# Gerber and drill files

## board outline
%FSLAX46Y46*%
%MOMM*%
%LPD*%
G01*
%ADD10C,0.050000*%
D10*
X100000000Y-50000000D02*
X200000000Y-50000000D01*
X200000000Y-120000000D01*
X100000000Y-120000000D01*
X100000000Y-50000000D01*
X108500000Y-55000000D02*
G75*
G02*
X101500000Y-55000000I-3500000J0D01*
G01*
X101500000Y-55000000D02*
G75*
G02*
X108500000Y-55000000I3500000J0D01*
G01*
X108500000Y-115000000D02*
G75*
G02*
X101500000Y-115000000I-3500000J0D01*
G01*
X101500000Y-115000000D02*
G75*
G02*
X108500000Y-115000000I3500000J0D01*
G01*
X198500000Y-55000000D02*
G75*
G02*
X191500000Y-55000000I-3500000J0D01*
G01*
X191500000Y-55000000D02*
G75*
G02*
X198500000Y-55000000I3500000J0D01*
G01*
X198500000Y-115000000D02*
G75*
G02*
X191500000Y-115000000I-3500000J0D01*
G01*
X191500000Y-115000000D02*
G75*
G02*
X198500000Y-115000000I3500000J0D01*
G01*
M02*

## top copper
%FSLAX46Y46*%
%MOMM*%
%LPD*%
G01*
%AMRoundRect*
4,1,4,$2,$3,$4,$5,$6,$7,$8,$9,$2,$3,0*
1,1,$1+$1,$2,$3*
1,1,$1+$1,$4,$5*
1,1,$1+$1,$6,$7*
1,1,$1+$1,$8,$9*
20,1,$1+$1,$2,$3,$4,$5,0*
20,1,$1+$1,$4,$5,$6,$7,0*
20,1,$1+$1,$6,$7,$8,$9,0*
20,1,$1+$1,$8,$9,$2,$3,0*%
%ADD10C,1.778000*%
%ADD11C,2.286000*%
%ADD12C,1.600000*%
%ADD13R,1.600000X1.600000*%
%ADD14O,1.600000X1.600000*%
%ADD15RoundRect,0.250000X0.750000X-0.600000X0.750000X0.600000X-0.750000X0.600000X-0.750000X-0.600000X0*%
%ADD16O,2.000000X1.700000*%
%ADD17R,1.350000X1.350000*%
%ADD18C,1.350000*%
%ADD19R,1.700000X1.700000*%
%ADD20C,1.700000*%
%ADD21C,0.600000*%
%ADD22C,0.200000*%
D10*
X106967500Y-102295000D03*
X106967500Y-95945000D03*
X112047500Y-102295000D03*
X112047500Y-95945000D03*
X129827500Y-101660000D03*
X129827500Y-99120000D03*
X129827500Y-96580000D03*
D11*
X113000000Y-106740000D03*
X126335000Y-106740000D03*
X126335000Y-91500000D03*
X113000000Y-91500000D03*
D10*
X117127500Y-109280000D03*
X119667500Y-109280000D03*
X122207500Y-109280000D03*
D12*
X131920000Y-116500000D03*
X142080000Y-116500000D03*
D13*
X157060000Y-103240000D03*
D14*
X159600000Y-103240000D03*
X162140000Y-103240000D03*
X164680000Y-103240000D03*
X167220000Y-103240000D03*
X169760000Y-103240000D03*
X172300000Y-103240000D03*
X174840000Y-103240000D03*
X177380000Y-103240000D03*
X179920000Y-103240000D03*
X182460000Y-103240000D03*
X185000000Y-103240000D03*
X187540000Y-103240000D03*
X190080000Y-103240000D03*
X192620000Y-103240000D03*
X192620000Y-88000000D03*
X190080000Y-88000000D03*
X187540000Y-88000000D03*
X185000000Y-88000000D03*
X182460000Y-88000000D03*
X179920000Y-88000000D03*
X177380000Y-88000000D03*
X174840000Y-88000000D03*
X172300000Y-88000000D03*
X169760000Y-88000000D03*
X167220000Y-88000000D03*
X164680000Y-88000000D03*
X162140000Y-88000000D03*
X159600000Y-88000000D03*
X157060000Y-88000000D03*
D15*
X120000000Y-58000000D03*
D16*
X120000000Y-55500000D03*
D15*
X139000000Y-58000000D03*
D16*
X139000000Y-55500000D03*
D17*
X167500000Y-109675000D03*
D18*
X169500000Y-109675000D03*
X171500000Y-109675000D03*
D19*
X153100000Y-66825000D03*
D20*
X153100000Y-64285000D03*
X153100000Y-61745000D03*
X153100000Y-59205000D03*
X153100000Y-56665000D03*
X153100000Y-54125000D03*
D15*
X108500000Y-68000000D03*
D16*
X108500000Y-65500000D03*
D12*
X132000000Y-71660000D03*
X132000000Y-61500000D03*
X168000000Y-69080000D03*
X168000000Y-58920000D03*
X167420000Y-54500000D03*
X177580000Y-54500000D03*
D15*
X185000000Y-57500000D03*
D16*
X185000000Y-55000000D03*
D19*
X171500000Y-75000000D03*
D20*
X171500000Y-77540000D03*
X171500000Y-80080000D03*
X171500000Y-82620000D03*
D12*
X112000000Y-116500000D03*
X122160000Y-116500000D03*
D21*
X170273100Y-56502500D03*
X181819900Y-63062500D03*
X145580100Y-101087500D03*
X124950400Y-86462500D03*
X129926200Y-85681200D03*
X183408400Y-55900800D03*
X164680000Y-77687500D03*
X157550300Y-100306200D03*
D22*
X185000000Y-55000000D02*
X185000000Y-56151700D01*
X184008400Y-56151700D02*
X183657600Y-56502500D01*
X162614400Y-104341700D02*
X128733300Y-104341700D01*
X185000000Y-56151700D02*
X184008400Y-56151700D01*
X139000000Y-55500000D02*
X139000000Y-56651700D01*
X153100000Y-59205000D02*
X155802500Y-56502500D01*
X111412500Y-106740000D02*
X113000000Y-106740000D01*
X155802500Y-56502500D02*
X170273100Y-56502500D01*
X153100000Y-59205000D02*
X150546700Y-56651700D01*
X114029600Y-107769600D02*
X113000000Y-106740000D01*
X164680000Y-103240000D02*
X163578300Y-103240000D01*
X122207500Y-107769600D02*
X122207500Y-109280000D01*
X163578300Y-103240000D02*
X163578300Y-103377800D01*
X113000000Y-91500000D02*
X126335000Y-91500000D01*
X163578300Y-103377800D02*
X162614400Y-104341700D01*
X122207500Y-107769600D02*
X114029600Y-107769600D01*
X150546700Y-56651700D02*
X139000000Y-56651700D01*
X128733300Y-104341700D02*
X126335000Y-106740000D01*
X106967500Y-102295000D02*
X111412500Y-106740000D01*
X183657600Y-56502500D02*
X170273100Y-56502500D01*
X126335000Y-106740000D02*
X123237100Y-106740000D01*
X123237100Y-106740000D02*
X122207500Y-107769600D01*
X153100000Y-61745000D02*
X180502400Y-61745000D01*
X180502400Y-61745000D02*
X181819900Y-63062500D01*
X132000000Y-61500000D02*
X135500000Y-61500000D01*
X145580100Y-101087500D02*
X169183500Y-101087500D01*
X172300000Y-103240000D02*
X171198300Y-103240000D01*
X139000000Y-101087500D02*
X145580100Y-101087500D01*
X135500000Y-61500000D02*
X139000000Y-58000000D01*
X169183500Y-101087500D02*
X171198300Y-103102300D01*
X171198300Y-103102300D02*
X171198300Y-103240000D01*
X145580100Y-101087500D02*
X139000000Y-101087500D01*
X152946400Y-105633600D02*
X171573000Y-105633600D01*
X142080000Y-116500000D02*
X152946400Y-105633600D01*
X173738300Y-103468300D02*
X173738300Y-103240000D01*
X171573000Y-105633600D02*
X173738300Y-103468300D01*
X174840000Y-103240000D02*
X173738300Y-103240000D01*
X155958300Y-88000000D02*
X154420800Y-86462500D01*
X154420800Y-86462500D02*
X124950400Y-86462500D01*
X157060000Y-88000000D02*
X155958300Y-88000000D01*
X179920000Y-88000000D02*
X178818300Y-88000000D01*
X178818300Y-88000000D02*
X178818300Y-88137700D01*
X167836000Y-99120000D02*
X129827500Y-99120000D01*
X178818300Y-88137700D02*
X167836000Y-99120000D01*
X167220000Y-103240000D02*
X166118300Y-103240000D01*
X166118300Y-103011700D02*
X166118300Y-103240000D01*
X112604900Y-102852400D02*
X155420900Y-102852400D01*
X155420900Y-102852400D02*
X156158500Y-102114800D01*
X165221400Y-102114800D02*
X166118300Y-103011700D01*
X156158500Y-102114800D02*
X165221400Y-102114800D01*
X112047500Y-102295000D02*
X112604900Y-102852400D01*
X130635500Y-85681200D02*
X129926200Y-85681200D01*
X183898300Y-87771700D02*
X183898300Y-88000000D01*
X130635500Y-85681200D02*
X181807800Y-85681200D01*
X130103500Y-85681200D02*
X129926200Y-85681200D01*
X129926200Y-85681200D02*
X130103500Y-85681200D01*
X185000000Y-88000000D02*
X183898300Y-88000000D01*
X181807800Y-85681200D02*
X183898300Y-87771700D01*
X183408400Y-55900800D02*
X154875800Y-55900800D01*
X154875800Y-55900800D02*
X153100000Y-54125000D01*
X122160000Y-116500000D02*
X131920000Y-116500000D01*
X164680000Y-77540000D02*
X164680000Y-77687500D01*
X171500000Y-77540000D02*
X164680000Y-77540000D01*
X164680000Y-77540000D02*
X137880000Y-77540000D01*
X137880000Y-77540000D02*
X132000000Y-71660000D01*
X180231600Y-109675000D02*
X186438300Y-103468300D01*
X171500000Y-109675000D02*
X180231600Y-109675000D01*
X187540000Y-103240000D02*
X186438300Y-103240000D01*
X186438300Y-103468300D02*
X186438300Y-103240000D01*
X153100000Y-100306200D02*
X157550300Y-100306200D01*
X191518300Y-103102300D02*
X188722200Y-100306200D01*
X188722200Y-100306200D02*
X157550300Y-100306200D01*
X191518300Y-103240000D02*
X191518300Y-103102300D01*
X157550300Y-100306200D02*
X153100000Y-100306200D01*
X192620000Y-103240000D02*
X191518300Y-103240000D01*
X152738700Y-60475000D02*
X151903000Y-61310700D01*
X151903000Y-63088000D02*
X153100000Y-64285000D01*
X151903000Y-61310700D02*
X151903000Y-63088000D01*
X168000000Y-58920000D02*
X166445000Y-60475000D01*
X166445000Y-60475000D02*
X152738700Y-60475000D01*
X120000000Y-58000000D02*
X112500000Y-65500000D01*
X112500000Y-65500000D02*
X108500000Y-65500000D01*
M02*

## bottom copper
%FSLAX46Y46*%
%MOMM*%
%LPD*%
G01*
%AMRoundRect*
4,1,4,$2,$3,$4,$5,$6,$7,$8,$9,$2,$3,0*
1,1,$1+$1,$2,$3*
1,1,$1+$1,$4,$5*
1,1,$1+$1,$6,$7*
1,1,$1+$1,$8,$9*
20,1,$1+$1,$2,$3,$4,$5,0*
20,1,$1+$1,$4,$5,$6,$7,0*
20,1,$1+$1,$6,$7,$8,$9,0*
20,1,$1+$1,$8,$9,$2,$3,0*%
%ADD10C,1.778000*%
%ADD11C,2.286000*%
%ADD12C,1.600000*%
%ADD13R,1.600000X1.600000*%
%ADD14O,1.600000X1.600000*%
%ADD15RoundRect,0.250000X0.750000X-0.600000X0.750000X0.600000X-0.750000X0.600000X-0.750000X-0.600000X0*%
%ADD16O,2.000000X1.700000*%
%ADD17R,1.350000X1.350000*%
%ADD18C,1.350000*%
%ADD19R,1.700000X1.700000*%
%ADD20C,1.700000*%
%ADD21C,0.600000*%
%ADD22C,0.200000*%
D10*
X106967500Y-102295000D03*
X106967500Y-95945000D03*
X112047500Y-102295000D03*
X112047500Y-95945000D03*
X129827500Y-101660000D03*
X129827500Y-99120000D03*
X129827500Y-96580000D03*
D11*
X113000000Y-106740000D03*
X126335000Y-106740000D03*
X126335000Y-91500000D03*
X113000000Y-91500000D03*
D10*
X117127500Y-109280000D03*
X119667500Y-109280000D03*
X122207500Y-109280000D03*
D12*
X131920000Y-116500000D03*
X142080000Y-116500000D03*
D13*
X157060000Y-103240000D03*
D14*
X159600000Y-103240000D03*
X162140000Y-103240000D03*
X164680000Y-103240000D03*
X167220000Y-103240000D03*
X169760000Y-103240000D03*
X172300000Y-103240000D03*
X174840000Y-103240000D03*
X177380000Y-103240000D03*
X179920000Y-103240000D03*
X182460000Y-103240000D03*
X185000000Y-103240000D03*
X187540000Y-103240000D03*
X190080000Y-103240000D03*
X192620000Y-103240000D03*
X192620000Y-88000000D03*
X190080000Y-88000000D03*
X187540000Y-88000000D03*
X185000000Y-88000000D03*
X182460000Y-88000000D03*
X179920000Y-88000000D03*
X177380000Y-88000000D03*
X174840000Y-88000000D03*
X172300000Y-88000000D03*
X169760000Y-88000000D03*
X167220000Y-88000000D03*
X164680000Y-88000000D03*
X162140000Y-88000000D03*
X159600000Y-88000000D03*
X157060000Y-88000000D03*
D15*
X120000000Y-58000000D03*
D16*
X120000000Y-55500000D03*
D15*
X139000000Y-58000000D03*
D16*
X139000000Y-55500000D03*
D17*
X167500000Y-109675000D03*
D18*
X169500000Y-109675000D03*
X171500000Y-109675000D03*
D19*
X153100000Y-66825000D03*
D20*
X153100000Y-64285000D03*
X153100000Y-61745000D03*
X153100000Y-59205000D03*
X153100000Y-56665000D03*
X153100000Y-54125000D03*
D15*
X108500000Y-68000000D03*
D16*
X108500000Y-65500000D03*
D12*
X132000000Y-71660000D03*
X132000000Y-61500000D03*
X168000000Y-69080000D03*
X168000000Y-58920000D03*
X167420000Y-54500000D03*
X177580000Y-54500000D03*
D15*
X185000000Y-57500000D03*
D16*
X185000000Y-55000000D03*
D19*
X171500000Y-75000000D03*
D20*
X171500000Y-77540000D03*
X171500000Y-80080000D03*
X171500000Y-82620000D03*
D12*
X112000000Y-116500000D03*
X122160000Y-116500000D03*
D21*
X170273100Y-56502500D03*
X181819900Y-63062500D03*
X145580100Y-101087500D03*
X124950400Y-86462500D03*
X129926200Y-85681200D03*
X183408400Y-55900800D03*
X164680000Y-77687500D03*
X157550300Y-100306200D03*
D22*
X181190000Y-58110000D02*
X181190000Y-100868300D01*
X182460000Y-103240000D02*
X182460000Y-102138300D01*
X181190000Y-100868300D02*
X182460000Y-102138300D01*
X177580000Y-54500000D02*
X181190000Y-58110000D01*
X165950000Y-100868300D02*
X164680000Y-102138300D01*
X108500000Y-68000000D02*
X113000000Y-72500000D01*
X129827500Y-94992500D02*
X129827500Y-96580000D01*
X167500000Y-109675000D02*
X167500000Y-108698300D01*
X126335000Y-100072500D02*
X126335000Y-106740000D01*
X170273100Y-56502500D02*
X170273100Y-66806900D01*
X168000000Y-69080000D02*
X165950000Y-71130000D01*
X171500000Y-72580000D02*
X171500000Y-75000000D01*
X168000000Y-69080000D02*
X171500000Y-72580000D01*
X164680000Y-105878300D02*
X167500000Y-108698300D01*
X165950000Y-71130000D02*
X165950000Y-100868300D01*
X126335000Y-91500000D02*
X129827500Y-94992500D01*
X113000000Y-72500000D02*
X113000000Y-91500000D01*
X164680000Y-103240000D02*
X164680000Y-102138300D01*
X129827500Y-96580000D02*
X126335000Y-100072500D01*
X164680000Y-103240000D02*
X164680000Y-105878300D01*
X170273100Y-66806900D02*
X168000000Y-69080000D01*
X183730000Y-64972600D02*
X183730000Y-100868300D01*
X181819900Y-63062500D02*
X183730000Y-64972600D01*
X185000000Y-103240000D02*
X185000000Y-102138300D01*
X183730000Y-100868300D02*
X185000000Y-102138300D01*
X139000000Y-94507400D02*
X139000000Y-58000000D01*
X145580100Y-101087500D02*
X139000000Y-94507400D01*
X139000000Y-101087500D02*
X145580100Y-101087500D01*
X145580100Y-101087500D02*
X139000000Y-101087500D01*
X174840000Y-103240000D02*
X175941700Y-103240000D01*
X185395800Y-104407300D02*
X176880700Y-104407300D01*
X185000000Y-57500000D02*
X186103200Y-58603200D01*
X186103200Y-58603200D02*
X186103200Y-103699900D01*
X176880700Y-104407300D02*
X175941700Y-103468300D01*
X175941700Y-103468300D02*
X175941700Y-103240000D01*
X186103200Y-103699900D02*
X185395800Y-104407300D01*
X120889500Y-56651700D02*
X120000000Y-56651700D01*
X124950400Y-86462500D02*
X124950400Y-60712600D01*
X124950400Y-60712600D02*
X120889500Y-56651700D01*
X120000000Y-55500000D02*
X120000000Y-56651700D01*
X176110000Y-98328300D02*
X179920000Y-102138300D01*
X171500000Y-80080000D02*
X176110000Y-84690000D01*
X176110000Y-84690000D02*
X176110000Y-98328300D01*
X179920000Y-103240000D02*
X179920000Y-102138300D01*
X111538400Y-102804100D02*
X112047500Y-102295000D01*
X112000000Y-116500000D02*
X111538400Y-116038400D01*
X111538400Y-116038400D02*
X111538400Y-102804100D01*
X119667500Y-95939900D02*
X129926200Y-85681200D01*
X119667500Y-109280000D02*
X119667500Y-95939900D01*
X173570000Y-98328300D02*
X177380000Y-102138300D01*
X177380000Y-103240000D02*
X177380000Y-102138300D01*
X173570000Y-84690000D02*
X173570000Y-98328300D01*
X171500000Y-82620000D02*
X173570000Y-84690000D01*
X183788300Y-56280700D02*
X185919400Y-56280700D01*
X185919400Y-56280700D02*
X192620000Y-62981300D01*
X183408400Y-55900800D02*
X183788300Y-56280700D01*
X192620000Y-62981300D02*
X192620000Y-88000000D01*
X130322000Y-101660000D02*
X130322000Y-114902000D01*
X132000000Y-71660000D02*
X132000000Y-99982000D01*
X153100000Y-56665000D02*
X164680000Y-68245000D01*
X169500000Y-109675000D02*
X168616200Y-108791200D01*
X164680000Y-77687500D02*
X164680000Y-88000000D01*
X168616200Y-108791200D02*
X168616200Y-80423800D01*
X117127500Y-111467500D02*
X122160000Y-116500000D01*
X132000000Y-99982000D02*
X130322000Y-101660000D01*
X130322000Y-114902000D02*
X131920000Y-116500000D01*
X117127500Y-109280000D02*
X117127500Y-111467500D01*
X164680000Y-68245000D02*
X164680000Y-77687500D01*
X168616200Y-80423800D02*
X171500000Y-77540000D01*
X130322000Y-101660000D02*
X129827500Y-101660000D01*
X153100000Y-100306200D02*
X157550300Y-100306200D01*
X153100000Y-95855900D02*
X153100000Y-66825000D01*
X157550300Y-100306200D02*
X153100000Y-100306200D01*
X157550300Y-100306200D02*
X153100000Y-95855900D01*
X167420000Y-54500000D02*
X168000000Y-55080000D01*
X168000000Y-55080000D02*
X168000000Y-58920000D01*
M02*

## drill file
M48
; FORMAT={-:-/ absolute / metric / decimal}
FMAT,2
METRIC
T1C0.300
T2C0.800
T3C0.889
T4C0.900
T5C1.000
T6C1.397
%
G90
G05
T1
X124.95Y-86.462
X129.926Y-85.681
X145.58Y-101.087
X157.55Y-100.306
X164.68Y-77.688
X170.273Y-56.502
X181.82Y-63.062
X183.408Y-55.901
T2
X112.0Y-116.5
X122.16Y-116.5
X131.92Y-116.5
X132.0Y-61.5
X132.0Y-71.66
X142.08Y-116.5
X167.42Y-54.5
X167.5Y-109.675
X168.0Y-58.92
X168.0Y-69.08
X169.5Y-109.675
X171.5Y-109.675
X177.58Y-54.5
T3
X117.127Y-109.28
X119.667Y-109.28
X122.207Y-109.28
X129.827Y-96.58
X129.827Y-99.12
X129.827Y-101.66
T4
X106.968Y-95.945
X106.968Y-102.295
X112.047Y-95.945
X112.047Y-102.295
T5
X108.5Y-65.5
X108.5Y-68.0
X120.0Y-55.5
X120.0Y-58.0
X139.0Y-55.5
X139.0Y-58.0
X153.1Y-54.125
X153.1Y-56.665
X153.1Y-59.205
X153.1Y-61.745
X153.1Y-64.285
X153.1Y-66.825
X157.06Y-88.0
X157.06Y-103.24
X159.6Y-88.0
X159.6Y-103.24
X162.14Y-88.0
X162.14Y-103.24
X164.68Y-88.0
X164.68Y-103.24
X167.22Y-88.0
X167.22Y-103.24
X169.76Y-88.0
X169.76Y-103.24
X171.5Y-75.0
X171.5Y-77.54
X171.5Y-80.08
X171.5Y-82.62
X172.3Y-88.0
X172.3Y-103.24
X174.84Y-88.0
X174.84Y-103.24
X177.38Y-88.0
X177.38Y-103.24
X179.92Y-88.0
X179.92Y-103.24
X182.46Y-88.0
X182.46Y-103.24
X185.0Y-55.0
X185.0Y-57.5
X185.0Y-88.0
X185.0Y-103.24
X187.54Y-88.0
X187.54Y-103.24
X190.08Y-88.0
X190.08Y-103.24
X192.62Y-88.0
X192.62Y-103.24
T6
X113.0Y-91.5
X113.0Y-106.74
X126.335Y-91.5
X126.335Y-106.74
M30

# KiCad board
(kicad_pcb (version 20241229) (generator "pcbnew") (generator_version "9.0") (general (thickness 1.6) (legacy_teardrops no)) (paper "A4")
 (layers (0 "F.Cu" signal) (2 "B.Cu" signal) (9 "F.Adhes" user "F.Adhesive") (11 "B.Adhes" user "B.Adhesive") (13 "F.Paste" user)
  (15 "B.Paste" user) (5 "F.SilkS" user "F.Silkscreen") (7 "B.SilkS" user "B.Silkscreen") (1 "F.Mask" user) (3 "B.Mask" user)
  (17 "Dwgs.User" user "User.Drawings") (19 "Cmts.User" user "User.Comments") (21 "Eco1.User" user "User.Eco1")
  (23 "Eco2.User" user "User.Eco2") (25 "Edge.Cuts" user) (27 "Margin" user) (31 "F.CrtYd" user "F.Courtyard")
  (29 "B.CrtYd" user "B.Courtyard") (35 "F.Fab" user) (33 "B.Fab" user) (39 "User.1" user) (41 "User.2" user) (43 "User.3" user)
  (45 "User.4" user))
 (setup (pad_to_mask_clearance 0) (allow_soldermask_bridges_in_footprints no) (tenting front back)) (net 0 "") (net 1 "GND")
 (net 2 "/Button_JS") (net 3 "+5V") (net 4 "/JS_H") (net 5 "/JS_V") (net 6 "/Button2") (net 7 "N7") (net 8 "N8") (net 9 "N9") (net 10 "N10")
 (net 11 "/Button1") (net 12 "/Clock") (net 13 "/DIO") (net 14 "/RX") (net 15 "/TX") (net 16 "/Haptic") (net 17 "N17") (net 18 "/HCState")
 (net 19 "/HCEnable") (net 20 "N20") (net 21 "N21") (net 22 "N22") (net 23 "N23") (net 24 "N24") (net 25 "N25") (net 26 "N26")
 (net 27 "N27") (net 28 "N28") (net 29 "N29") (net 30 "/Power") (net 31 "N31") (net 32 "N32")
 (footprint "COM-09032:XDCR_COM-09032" (layer "F.Cu") (at 119.6675 99.12 90)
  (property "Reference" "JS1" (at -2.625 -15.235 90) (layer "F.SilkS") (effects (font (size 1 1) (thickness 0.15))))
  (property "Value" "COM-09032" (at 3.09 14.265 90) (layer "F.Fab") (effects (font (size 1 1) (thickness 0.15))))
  (pad "B1A" thru_hole circle (at -3.175 -12.7 90) (size 1.778 1.778) (drill 0.9) (layers "*.Cu" "*.Mask") (remove_unused_layers no)
   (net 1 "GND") (solder_mask_margin 0.102))
  (pad "B1B" thru_hole circle (at 3.175 -12.7 90) (size 1.778 1.778) (drill 0.9) (layers "*.Cu" "*.Mask") (remove_unused_layers no)
   (solder_mask_margin 0.102))
  (pad "B2A" thru_hole circle (at -3.175 -7.62 90) (size 1.778 1.778) (drill 0.9) (layers "*.Cu" "*.Mask") (remove_unused_layers no)
   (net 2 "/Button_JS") (solder_mask_margin 0.102))
  (pad "B2B" thru_hole circle (at 3.175 -7.62 90) (size 1.778 1.778) (drill 0.9) (layers "*.Cu" "*.Mask") (remove_unused_layers no)
   (solder_mask_margin 0.102))
  (pad "H1" thru_hole circle (at -2.54 10.16 90) (size 1.778 1.778) (drill 0.889) (layers "*.Cu" "*.Mask") (remove_unused_layers no)
   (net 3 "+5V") (solder_mask_margin 0.102))
  (pad "H2" thru_hole circle (at 0 10.16 90) (size 1.778 1.778) (drill 0.889) (layers "*.Cu" "*.Mask") (remove_unused_layers no)
   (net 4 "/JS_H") (solder_mask_margin 0.102))
  (pad "H3" thru_hole circle (at 2.54 10.16 90) (size 1.778 1.778) (drill 0.889) (layers "*.Cu" "*.Mask") (remove_unused_layers no)
   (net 1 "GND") (solder_mask_margin 0.102))
  (pad "S1" thru_hole circle (at -7.62 -6.6675 90) (size 2.286 2.286) (drill 1.397) (layers "*.Cu" "*.Mask") (remove_unused_layers no)
   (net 1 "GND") (solder_mask_margin 0.102))
  (pad "S2" thru_hole circle (at -7.62 6.6675 90) (size 2.286 2.286) (drill 1.397) (layers "*.Cu" "*.Mask") (remove_unused_layers no)
   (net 1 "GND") (solder_mask_margin 0.102))
  (pad "S3" thru_hole circle (at 7.62 6.6675 90) (size 2.286 2.286) (drill 1.397) (layers "*.Cu" "*.Mask") (remove_unused_layers no)
   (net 1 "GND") (solder_mask_margin 0.102))
  (pad "S4" thru_hole circle (at 7.62 -6.6675 90) (size 2.286 2.286) (drill 1.397) (layers "*.Cu" "*.Mask") (remove_unused_layers no)
   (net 1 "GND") (solder_mask_margin 0.102))
  (pad "V1" thru_hole circle (at -10.16 -2.54 90) (size 1.778 1.778) (drill 0.889) (layers "*.Cu" "*.Mask") (remove_unused_layers no)
   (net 3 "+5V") (solder_mask_margin 0.102))
  (pad "V2" thru_hole circle (at -10.16 0 90) (size 1.778 1.778) (drill 0.889) (layers "*.Cu" "*.Mask") (remove_unused_layers no)
   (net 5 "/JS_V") (solder_mask_margin 0.102))
  (pad "V3" thru_hole circle (at -10.16 2.54 90) (size 1.778 1.778) (drill 0.889) (layers "*.Cu" "*.Mask") (remove_unused_layers no)
   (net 1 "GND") (solder_mask_margin 0.102)))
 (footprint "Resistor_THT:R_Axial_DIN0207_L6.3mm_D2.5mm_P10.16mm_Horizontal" (layer "F.Cu") (at 131.92 116.5)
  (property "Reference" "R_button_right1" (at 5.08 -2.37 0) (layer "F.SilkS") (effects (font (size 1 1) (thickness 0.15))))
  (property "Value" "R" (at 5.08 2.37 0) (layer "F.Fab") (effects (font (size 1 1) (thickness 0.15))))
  (pad "1" thru_hole circle (at 0 0) (size 1.6 1.6) (drill 0.8) (layers "*.Cu" "*.Mask") (remove_unused_layers no) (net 3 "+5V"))
  (pad "2" thru_hole circle (at 10.16 0) (size 1.6 1.6) (drill 0.8) (layers "*.Cu" "*.Mask") (remove_unused_layers no) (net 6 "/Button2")))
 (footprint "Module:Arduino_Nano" (layer "F.Cu") (at 157.06 103.24 90)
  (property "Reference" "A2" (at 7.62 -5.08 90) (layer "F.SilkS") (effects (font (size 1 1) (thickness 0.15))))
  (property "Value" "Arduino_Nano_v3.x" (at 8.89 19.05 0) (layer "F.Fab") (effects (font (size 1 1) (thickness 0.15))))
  (pad "1" thru_hole rect (at 0 0 90) (size 1.6 1.6) (drill 1) (layers "*.Cu" "*.Mask") (remove_unused_layers no) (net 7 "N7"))
  (pad "2" thru_hole oval (at 0 2.54 90) (size 1.6 1.6) (drill 1) (layers "*.Cu" "*.Mask") (remove_unused_layers no) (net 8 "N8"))
  (pad "3" thru_hole oval (at 0 5.08 90) (size 1.6 1.6) (drill 1) (layers "*.Cu" "*.Mask") (remove_unused_layers no) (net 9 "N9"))
  (pad "4" thru_hole oval (at 0 7.62 90) (size 1.6 1.6) (drill 1) (layers "*.Cu" "*.Mask") (remove_unused_layers no) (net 1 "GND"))
  (pad "5" thru_hole oval (at 0 10.16 90) (size 1.6 1.6) (drill 1) (layers "*.Cu" "*.Mask") (remove_unused_layers no) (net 2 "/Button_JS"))
  (pad "6" thru_hole oval (at 0 12.7 90) (size 1.6 1.6) (drill 1) (layers "*.Cu" "*.Mask") (remove_unused_layers no) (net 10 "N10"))
  (pad "7" thru_hole oval (at 0 15.24 90) (size 1.6 1.6) (drill 1) (layers "*.Cu" "*.Mask") (remove_unused_layers no) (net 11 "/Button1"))
  (pad "8" thru_hole oval (at 0 17.78 90) (size 1.6 1.6) (drill 1) (layers "*.Cu" "*.Mask") (remove_unused_layers no) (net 6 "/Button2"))
  (pad "9" thru_hole oval (at 0 20.32 90) (size 1.6 1.6) (drill 1) (layers "*.Cu" "*.Mask") (remove_unused_layers no) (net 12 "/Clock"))
  (pad "10" thru_hole oval (at 0 22.86 90) (size 1.6 1.6) (drill 1) (layers "*.Cu" "*.Mask") (remove_unused_layers no) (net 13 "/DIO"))
  (pad "11" thru_hole oval (at 0 25.4 90) (size 1.6 1.6) (drill 1) (layers "*.Cu" "*.Mask") (remove_unused_layers no) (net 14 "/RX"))
  (pad "12" thru_hole oval (at 0 27.94 90) (size 1.6 1.6) (drill 1) (layers "*.Cu" "*.Mask") (remove_unused_layers no) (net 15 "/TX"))
  (pad "13" thru_hole oval (at 0 30.48 90) (size 1.6 1.6) (drill 1) (layers "*.Cu" "*.Mask") (remove_unused_layers no) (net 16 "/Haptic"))
  (pad "14" thru_hole oval (at 0 33.02 90) (size 1.6 1.6) (drill 1) (layers "*.Cu" "*.Mask") (remove_unused_layers no) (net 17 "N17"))
  (pad "15" thru_hole oval (at 0 35.56 90) (size 1.6 1.6) (drill 1) (layers "*.Cu" "*.Mask") (remove_unused_layers no) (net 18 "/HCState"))
  (pad "16" thru_hole oval (at 15.24 35.56 90) (size 1.6 1.6) (drill 1) (layers "*.Cu" "*.Mask") (remove_unused_layers no)
   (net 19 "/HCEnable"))
  (pad "17" thru_hole oval (at 15.24 33.02 90) (size 1.6 1.6) (drill 1) (layers "*.Cu" "*.Mask") (remove_unused_layers no) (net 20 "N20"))
  (pad "18" thru_hole oval (at 15.24 30.48 90) (size 1.6 1.6) (drill 1) (layers "*.Cu" "*.Mask") (remove_unused_layers no) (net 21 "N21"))
  (pad "19" thru_hole oval (at 15.24 27.94 90) (size 1.6 1.6) (drill 1) (layers "*.Cu" "*.Mask") (remove_unused_layers no) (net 5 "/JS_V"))
  (pad "20" thru_hole oval (at 15.24 25.4 90) (size 1.6 1.6) (drill 1) (layers "*.Cu" "*.Mask") (remove_unused_layers no) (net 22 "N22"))
  (pad "21" thru_hole oval (at 15.24 22.86 90) (size 1.6 1.6) (drill 1) (layers "*.Cu" "*.Mask") (remove_unused_layers no) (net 4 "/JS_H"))
  (pad "22" thru_hole oval (at 15.24 20.32 90) (size 1.6 1.6) (drill 1) (layers "*.Cu" "*.Mask") (remove_unused_layers no) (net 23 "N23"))
  (pad "23" thru_hole oval (at 15.24 17.78 90) (size 1.6 1.6) (drill 1) (layers "*.Cu" "*.Mask") (remove_unused_layers no) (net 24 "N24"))
  (pad "24" thru_hole oval (at 15.24 15.24 90) (size 1.6 1.6) (drill 1) (layers "*.Cu" "*.Mask") (remove_unused_layers no) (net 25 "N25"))
  (pad "25" thru_hole oval (at 15.24 12.7 90) (size 1.6 1.6) (drill 1) (layers "*.Cu" "*.Mask") (remove_unused_layers no) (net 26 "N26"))
  (pad "26" thru_hole oval (at 15.24 10.16 90) (size 1.6 1.6) (drill 1) (layers "*.Cu" "*.Mask") (remove_unused_layers no) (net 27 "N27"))
  (pad "27" thru_hole oval (at 15.24 7.62 90) (size 1.6 1.6) (drill 1) (layers "*.Cu" "*.Mask") (remove_unused_layers no) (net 3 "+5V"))
  (pad "28" thru_hole oval (at 15.24 5.08 90) (size 1.6 1.6) (drill 1) (layers "*.Cu" "*.Mask") (remove_unused_layers no) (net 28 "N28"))
  (pad "29" thru_hole oval (at 15.24 2.54 90) (size 1.6 1.6) (drill 1) (layers "*.Cu" "*.Mask") (remove_unused_layers no) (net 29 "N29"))
  (pad "30" thru_hole oval (at 15.24 0 90) (size 1.6 1.6) (drill 1) (layers "*.Cu" "*.Mask") (remove_unused_layers no) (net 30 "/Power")))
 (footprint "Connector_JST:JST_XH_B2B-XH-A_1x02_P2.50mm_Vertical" (layer "F.Cu") (at 120 58 90)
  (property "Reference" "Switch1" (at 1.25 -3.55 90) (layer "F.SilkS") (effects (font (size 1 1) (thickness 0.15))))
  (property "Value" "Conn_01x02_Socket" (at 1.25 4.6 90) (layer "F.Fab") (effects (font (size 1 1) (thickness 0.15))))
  (pad "1" thru_hole roundrect (at 0 0 90) (size 1.7 2) (drill 1) (layers "*.Cu" "*.Mask") (remove_unused_layers no)
   (roundrect_rratio 0.147059) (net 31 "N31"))
  (pad "2" thru_hole oval (at 2.5 0 90) (size 1.7 2) (drill 1) (layers "*.Cu" "*.Mask") (remove_unused_layers no) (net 30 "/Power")))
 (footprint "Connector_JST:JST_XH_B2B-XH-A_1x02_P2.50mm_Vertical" (layer "F.Cu") (at 139 58 90)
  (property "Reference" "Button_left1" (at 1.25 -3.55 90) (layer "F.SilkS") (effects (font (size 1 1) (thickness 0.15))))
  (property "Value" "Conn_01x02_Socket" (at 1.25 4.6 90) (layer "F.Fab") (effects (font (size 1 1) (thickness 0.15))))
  (pad "1" thru_hole roundrect (at 0 0 90) (size 1.7 2) (drill 1) (layers "*.Cu" "*.Mask") (remove_unused_layers no)
   (roundrect_rratio 0.147059) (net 11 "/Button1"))
  (pad "2" thru_hole oval (at 2.5 0 90) (size 1.7 2) (drill 1) (layers "*.Cu" "*.Mask") (remove_unused_layers no) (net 1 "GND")))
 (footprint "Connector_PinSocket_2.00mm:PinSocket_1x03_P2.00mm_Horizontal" (layer "F.Cu") (at 167.5 109.675 90)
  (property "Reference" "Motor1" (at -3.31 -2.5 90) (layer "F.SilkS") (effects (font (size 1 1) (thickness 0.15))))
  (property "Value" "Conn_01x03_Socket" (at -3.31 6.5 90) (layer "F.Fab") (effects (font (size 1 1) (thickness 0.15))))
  (pad "1" thru_hole rect (at 0 0 90) (size 1.35 1.35) (drill 0.8) (layers "*.Cu" "*.Mask") (remove_unused_layers no) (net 1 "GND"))
  (pad "2" thru_hole circle (at 0 2 90) (size 1.35 1.35) (drill 0.8) (layers "*.Cu" "*.Mask") (remove_unused_layers no) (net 3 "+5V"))
  (pad "3" thru_hole circle (at 0 4 90) (size 1.35 1.35) (drill 0.8) (layers "*.Cu" "*.Mask") (remove_unused_layers no) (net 16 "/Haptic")))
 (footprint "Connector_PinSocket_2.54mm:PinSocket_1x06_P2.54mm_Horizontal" (layer "F.Cu") (at 153.1 66.825 180)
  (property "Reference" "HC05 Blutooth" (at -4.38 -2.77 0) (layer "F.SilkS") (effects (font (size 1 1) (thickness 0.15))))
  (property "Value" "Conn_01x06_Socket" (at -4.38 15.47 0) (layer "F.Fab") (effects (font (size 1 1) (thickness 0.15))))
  (pad "1" thru_hole rect (at 0 0 180) (size 1.7 1.7) (drill 1) (layers "*.Cu" "*.Mask") (remove_unused_layers no) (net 18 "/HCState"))
  (pad "2" thru_hole circle (at 0 2.54 180) (size 1.7 1.7) (drill 1) (layers "*.Cu" "*.Mask") (remove_unused_layers no) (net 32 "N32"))
  (pad "3" thru_hole circle (at 0 5.08 180) (size 1.7 1.7) (drill 1) (layers "*.Cu" "*.Mask") (remove_unused_layers no) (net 15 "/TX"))
  (pad "4" thru_hole circle (at 0 7.62 180) (size 1.7 1.7) (drill 1) (layers "*.Cu" "*.Mask") (remove_unused_layers no) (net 1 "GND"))
  (pad "5" thru_hole circle (at 0 10.16 180) (size 1.7 1.7) (drill 1) (layers "*.Cu" "*.Mask") (remove_unused_layers no) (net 3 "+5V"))
  (pad "6" thru_hole circle (at 0 12.7 180) (size 1.7 1.7) (drill 1) (layers "*.Cu" "*.Mask") (remove_unused_layers no) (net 19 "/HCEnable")))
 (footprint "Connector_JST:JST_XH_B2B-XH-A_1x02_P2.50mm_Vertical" (layer "F.Cu") (at 108.5 68 90)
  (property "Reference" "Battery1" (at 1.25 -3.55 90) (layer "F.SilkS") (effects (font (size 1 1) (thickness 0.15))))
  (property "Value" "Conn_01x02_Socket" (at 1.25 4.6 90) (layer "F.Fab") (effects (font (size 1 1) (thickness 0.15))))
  (pad "1" thru_hole roundrect (at 0 0 90) (size 1.7 2) (drill 1) (layers "*.Cu" "*.Mask") (remove_unused_layers no)
   (roundrect_rratio 0.147059) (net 1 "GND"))
  (pad "2" thru_hole oval (at 2.5 0 90) (size 1.7 2) (drill 1) (layers "*.Cu" "*.Mask") (remove_unused_layers no) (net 31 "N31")))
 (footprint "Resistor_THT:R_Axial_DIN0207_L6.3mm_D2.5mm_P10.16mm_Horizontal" (layer "F.Cu") (at 132 71.66 90)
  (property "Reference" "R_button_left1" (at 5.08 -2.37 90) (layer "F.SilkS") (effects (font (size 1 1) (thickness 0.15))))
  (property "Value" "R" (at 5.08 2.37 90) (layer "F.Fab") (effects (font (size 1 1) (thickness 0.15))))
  (pad "1" thru_hole circle (at 0 0 90) (size 1.6 1.6) (drill 0.8) (layers "*.Cu" "*.Mask") (remove_unused_layers no) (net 3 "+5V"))
  (pad "2" thru_hole circle (at 10.16 0 90) (size 1.6 1.6) (drill 0.8) (layers "*.Cu" "*.Mask") (remove_unused_layers no)
   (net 11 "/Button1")))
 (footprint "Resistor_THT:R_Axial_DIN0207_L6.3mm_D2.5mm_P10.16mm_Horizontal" (layer "F.Cu") (at 168 69.08 90)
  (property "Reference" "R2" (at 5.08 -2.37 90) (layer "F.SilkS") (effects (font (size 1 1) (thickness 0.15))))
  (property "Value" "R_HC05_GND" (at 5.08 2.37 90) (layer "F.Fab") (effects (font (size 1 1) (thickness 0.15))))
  (pad "1" thru_hole circle (at 0 0 90) (size 1.6 1.6) (drill 0.8) (layers "*.Cu" "*.Mask") (remove_unused_layers no) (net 1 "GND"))
  (pad "2" thru_hole circle (at 10.16 0 90) (size 1.6 1.6) (drill 0.8) (layers "*.Cu" "*.Mask") (remove_unused_layers no) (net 32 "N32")))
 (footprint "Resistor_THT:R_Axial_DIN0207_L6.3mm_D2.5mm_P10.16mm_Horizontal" (layer "F.Cu") (at 167.42 54.5)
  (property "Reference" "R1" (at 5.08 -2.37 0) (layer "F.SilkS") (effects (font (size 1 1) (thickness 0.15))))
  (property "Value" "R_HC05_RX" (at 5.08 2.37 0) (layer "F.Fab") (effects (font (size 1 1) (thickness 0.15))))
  (pad "1" thru_hole circle (at 0 0) (size 1.6 1.6) (drill 0.8) (layers "*.Cu" "*.Mask") (remove_unused_layers no) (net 32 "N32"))
  (pad "2" thru_hole circle (at 10.16 0) (size 1.6 1.6) (drill 0.8) (layers "*.Cu" "*.Mask") (remove_unused_layers no) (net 14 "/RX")))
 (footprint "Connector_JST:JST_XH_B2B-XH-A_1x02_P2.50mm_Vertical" (layer "F.Cu") (at 185 57.5 90)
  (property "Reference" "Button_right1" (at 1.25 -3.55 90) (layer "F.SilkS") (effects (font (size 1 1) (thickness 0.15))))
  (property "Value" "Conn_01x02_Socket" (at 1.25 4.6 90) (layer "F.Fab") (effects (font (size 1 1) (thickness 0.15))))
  (pad "1" thru_hole roundrect (at 0 0 90) (size 1.7 2) (drill 1) (layers "*.Cu" "*.Mask") (remove_unused_layers no)
   (roundrect_rratio 0.147059) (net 6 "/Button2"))
  (pad "2" thru_hole oval (at 2.5 0 90) (size 1.7 2) (drill 1) (layers "*.Cu" "*.Mask") (remove_unused_layers no) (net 1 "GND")))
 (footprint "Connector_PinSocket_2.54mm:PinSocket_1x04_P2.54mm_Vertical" (layer "F.Cu") (at 171.5 75)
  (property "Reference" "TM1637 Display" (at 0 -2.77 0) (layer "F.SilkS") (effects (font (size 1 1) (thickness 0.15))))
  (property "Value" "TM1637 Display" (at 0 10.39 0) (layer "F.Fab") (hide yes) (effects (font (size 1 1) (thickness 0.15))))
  (pad "1" thru_hole rect (at 0 0) (size 1.7 1.7) (drill 1) (layers "*.Cu" "*.Mask") (remove_unused_layers no) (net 1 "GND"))
  (pad "2" thru_hole circle (at 0 2.54) (size 1.7 1.7) (drill 1) (layers "*.Cu" "*.Mask") (remove_unused_layers no) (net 3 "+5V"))
  (pad "3" thru_hole circle (at 0 5.08) (size 1.7 1.7) (drill 1) (layers "*.Cu" "*.Mask") (remove_unused_layers no) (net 13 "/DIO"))
  (pad "4" thru_hole circle (at 0 7.62) (size 1.7 1.7) (drill 1) (layers "*.Cu" "*.Mask") (remove_unused_layers no) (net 12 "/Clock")))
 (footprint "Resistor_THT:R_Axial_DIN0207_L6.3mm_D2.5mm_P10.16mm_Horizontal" (layer "F.Cu") (at 112 116.5)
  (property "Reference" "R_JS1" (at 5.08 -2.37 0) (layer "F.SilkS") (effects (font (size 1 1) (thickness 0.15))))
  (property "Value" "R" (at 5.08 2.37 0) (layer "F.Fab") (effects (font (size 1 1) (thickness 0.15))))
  (pad "1" thru_hole circle (at 0 0) (size 1.6 1.6) (drill 0.8) (layers "*.Cu" "*.Mask") (remove_unused_layers no) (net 2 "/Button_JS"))
  (pad "2" thru_hole circle (at 10.16 0) (size 1.6 1.6) (drill 0.8) (layers "*.Cu" "*.Mask") (remove_unused_layers no) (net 3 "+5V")))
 (gr_rect (start 100 50) (end 200 120) (stroke (width 0.05) (type solid)) (fill no) (layer "Edge.Cuts"))
 (gr_circle (center 105 55) (end 108.5 55) (stroke (width 0.05) (type solid)) (fill no) (layer "Edge.Cuts"))
 (gr_circle (center 105 115) (end 108.5 115) (stroke (width 0.05) (type solid)) (fill no) (layer "Edge.Cuts"))
 (gr_circle (center 195 55) (end 198.5 55) (stroke (width 0.05) (type solid)) (fill no) (layer "Edge.Cuts"))
 (gr_circle (center 195 115) (end 198.5 115) (stroke (width 0.05) (type solid)) (fill no) (layer "Edge.Cuts"))
 (segment (start 181.19 58.11) (end 181.19 100.8683) (width 0.2) (layer "B.Cu") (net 14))
 (segment (start 182.46 103.24) (end 182.46 102.1383) (width 0.2) (layer "B.Cu") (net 14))
 (segment (start 181.19 100.8683) (end 182.46 102.1383) (width 0.2) (layer "B.Cu") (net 14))
 (segment (start 177.58 54.5) (end 181.19 58.11) (width 0.2) (layer "B.Cu") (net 14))
 (segment (start 185 55) (end 185 56.1517) (width 0.2) (layer "F.Cu") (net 1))
 (segment (start 184.0084 56.1517) (end 183.6576 56.5025) (width 0.2) (layer "F.Cu") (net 1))
 (segment (start 162.6144 104.3417) (end 128.7333 104.3417) (width 0.2) (layer "F.Cu") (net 1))
 (segment (start 185 56.1517) (end 184.0084 56.1517) (width 0.2) (layer "F.Cu") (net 1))
 (segment (start 139 55.5) (end 139 56.6517) (width 0.2) (layer "F.Cu") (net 1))
 (segment (start 153.1 59.205) (end 155.8025 56.5025) (width 0.2) (layer "F.Cu") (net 1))
 (segment (start 111.4125 106.74) (end 113 106.74) (width 0.2) (layer "F.Cu") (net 1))
 (segment (start 155.8025 56.5025) (end 170.2731 56.5025) (width 0.2) (layer "F.Cu") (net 1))
 (segment (start 153.1 59.205) (end 150.5467 56.6517) (width 0.2) (layer "F.Cu") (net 1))
 (segment (start 114.0296 107.7696) (end 113 106.74) (width 0.2) (layer "F.Cu") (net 1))
 (segment (start 164.68 103.24) (end 163.5783 103.24) (width 0.2) (layer "F.Cu") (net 1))
 (segment (start 122.2075 107.7696) (end 122.2075 109.28) (width 0.2) (layer "F.Cu") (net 1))
 (segment (start 163.5783 103.24) (end 163.5783 103.3778) (width 0.2) (layer "F.Cu") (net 1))
 (segment (start 113 91.5) (end 126.335 91.5) (width 0.2) (layer "F.Cu") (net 1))
 (segment (start 163.5783 103.3778) (end 162.6144 104.3417) (width 0.2) (layer "F.Cu") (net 1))
 (segment (start 122.2075 107.7696) (end 114.0296 107.7696) (width 0.2) (layer "F.Cu") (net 1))
 (segment (start 150.5467 56.6517) (end 139 56.6517) (width 0.2) (layer "F.Cu") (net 1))
 (segment (start 128.7333 104.3417) (end 126.335 106.74) (width 0.2) (layer "F.Cu") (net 1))
 (segment (start 106.9675 102.295) (end 111.4125 106.74) (width 0.2) (layer "F.Cu") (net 1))
 (segment (start 183.6576 56.5025) (end 170.2731 56.5025) (width 0.2) (layer "F.Cu") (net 1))
 (segment (start 126.335 106.74) (end 123.2371 106.74) (width 0.2) (layer "F.Cu") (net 1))
 (segment (start 123.2371 106.74) (end 122.2075 107.7696) (width 0.2) (layer "F.Cu") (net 1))
 (via (at 170.2731 56.5025) (size 0.6) (drill 0.3) (layers "F.Cu" "B.Cu") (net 1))
 (segment (start 165.95 100.8683) (end 164.68 102.1383) (width 0.2) (layer "B.Cu") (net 1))
 (segment (start 108.5 68) (end 113 72.5) (width 0.2) (layer "B.Cu") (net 1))
 (segment (start 129.8275 94.9925) (end 129.8275 96.58) (width 0.2) (layer "B.Cu") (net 1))
 (segment (start 167.5 109.675) (end 167.5 108.6983) (width 0.2) (layer "B.Cu") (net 1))
 (segment (start 126.335 100.0725) (end 126.335 106.74) (width 0.2) (layer "B.Cu") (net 1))
 (segment (start 170.2731 56.5025) (end 170.2731 66.8069) (width 0.2) (layer "B.Cu") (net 1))
 (segment (start 168 69.08) (end 165.95 71.13) (width 0.2) (layer "B.Cu") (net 1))
 (segment (start 171.5 72.58) (end 171.5 75) (width 0.2) (layer "B.Cu") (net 1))
 (segment (start 168 69.08) (end 171.5 72.58) (width 0.2) (layer "B.Cu") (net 1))
 (segment (start 164.68 105.8783) (end 167.5 108.6983) (width 0.2) (layer "B.Cu") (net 1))
 (segment (start 165.95 71.13) (end 165.95 100.8683) (width 0.2) (layer "B.Cu") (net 1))
 (segment (start 126.335 91.5) (end 129.8275 94.9925) (width 0.2) (layer "B.Cu") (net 1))
 (segment (start 113 72.5) (end 113 91.5) (width 0.2) (layer "B.Cu") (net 1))
 (segment (start 164.68 103.24) (end 164.68 102.1383) (width 0.2) (layer "B.Cu") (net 1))
 (segment (start 129.8275 96.58) (end 126.335 100.0725) (width 0.2) (layer "B.Cu") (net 1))
 (segment (start 164.68 103.24) (end 164.68 105.8783) (width 0.2) (layer "B.Cu") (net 1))
 (segment (start 170.2731 66.8069) (end 168 69.08) (width 0.2) (layer "B.Cu") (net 1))
 (segment (start 153.1 61.745) (end 180.5024 61.745) (width 0.2) (layer "F.Cu") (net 15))
 (segment (start 180.5024 61.745) (end 181.8199 63.0625) (width 0.2) (layer "F.Cu") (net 15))
 (via (at 181.8199 63.0625) (size 0.6) (drill 0.3) (layers "F.Cu" "B.Cu") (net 15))
 (segment (start 183.73 64.9726) (end 183.73 100.8683) (width 0.2) (layer "B.Cu") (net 15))
 (segment (start 181.8199 63.0625) (end 183.73 64.9726) (width 0.2) (layer "B.Cu") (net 15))
 (segment (start 185 103.24) (end 185 102.1383) (width 0.2) (layer "B.Cu") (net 15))
 (segment (start 183.73 100.8683) (end 185 102.1383) (width 0.2) (layer "B.Cu") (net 15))
 (segment (start 132 61.5) (end 135.5 61.5) (width 0.2) (layer "F.Cu") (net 11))
 (segment (start 145.5801 101.0875) (end 169.1835 101.0875) (width 0.2) (layer "F.Cu") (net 11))
 (segment (start 172.3 103.24) (end 171.1983 103.24) (width 0.2) (layer "F.Cu") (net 11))
 (segment (start 139 101.0875) (end 145.5801 101.0875) (width 0.2) (layer "F.Cu") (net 11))
 (segment (start 135.5 61.5) (end 139 58) (width 0.2) (layer "F.Cu") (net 11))
 (segment (start 169.1835 101.0875) (end 171.1983 103.1023) (width 0.2) (layer "F.Cu") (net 11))
 (segment (start 171.1983 103.1023) (end 171.1983 103.24) (width 0.2) (layer "F.Cu") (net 11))
 (segment (start 145.5801 101.0875) (end 139 101.0875) (width 0.2) (layer "F.Cu") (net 11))
 (via (at 145.5801 101.0875) (size 0.6) (drill 0.3) (layers "F.Cu" "B.Cu") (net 11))
 (segment (start 139 94.5074) (end 139 58) (width 0.2) (layer "B.Cu") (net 11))
 (segment (start 145.5801 101.0875) (end 139 94.5074) (width 0.2) (layer "B.Cu") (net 11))
 (segment (start 139 101.0875) (end 145.5801 101.0875) (width 0.2) (layer "B.Cu") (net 11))
 (segment (start 145.5801 101.0875) (end 139 101.0875) (width 0.2) (layer "B.Cu") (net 11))
 (segment (start 152.9464 105.6336) (end 171.573 105.6336) (width 0.2) (layer "F.Cu") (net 6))
 (segment (start 142.08 116.5) (end 152.9464 105.6336) (width 0.2) (layer "F.Cu") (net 6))
 (segment (start 173.7383 103.4683) (end 173.7383 103.24) (width 0.2) (layer "F.Cu") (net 6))
 (segment (start 171.573 105.6336) (end 173.7383 103.4683) (width 0.2) (layer "F.Cu") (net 6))
 (segment (start 174.84 103.24) (end 173.7383 103.24) (width 0.2) (layer "F.Cu") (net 6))
 (segment (start 174.84 103.24) (end 175.9417 103.24) (width 0.2) (layer "B.Cu") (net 6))
 (segment (start 185.3958 104.4073) (end 176.8807 104.4073) (width 0.2) (layer "B.Cu") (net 6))
 (segment (start 185 57.5) (end 186.1032 58.6032) (width 0.2) (layer "B.Cu") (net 6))
 (segment (start 186.1032 58.6032) (end 186.1032 103.6999) (width 0.2) (layer "B.Cu") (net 6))
 (segment (start 176.8807 104.4073) (end 175.9417 103.4683) (width 0.2) (layer "B.Cu") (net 6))
 (segment (start 175.9417 103.4683) (end 175.9417 103.24) (width 0.2) (layer "B.Cu") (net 6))
 (segment (start 186.1032 103.6999) (end 185.3958 104.4073) (width 0.2) (layer "B.Cu") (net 6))
 (segment (start 155.9583 88) (end 154.4208 86.4625) (width 0.2) (layer "F.Cu") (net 30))
 (segment (start 154.4208 86.4625) (end 124.9504 86.4625) (width 0.2) (layer "F.Cu") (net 30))
 (segment (start 157.06 88) (end 155.9583 88) (width 0.2) (layer "F.Cu") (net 30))
 (via (at 124.9504 86.4625) (size 0.6) (drill 0.3) (layers "F.Cu" "B.Cu") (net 30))
 (segment (start 120.8895 56.6517) (end 120 56.6517) (width 0.2) (layer "B.Cu") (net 30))
 (segment (start 124.9504 86.4625) (end 124.9504 60.7126) (width 0.2) (layer "B.Cu") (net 30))
 (segment (start 124.9504 60.7126) (end 120.8895 56.6517) (width 0.2) (layer "B.Cu") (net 30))
 (segment (start 120 55.5) (end 120 56.6517) (width 0.2) (layer "B.Cu") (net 30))
 (segment (start 176.11 98.3283) (end 179.92 102.1383) (width 0.2) (layer "B.Cu") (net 13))
 (segment (start 171.5 80.08) (end 176.11 84.69) (width 0.2) (layer "B.Cu") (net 13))
 (segment (start 176.11 84.69) (end 176.11 98.3283) (width 0.2) (layer "B.Cu") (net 13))
 (segment (start 179.92 103.24) (end 179.92 102.1383) (width 0.2) (layer "B.Cu") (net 13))
 (segment (start 179.92 88) (end 178.8183 88) (width 0.2) (layer "F.Cu") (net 4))
 (segment (start 178.8183 88) (end 178.8183 88.1377) (width 0.2) (layer "F.Cu") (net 4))
 (segment (start 167.836 99.12) (end 129.8275 99.12) (width 0.2) (layer "F.Cu") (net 4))
 (segment (start 178.8183 88.1377) (end 167.836 99.12) (width 0.2) (layer "F.Cu") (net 4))
 (segment (start 167.22 103.24) (end 166.1183 103.24) (width 0.2) (layer "F.Cu") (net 2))
 (segment (start 166.1183 103.0117) (end 166.1183 103.24) (width 0.2) (layer "F.Cu") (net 2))
 (segment (start 112.6049 102.8524) (end 155.4209 102.8524) (width 0.2) (layer "F.Cu") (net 2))
 (segment (start 155.4209 102.8524) (end 156.1585 102.1148) (width 0.2) (layer "F.Cu") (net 2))
 (segment (start 165.2214 102.1148) (end 166.1183 103.0117) (width 0.2) (layer "F.Cu") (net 2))
 (segment (start 156.1585 102.1148) (end 165.2214 102.1148) (width 0.2) (layer "F.Cu") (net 2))
 (segment (start 112.0475 102.295) (end 112.6049 102.8524) (width 0.2) (layer "F.Cu") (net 2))
 (segment (start 111.5384 102.8041) (end 112.0475 102.295) (width 0.2) (layer "B.Cu") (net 2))
 (segment (start 112 116.5) (end 111.5384 116.0384) (width 0.2) (layer "B.Cu") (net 2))
 (segment (start 111.5384 116.0384) (end 111.5384 102.8041) (width 0.2) (layer "B.Cu") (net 2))
 (segment (start 130.6355 85.6812) (end 129.9262 85.6812) (width 0.2) (layer "F.Cu") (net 5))
 (segment (start 183.8983 87.7717) (end 183.8983 88) (width 0.2) (layer "F.Cu") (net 5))
 (segment (start 130.6355 85.6812) (end 181.8078 85.6812) (width 0.2) (layer "F.Cu") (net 5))
 (segment (start 130.1035 85.6812) (end 129.9262 85.6812) (width 0.2) (layer "F.Cu") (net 5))
 (segment (start 129.9262 85.6812) (end 130.1035 85.6812) (width 0.2) (layer "F.Cu") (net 5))
 (segment (start 185 88) (end 183.8983 88) (width 0.2) (layer "F.Cu") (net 5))
 (segment (start 181.8078 85.6812) (end 183.8983 87.7717) (width 0.2) (layer "F.Cu") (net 5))
 (via (at 129.9262 85.6812) (size 0.6) (drill 0.3) (layers "F.Cu" "B.Cu") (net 5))
 (segment (start 119.6675 95.9399) (end 129.9262 85.6812) (width 0.2) (layer "B.Cu") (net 5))
 (segment (start 119.6675 109.28) (end 119.6675 95.9399) (width 0.2) (layer "B.Cu") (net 5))
 (segment (start 173.57 98.3283) (end 177.38 102.1383) (width 0.2) (layer "B.Cu") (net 12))
 (segment (start 177.38 103.24) (end 177.38 102.1383) (width 0.2) (layer "B.Cu") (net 12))
 (segment (start 173.57 84.69) (end 173.57 98.3283) (width 0.2) (layer "B.Cu") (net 12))
 (segment (start 171.5 82.62) (end 173.57 84.69) (width 0.2) (layer "B.Cu") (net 12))
 (segment (start 183.4084 55.9008) (end 154.8758 55.9008) (width 0.2) (layer "F.Cu") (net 19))
 (segment (start 154.8758 55.9008) (end 153.1 54.125) (width 0.2) (layer "F.Cu") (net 19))
 (via (at 183.4084 55.9008) (size 0.6) (drill 0.3) (layers "F.Cu" "B.Cu") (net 19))
 (segment (start 183.7883 56.2807) (end 185.9194 56.2807) (width 0.2) (layer "B.Cu") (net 19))
 (segment (start 185.9194 56.2807) (end 192.62 62.9813) (width 0.2) (layer "B.Cu") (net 19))
 (segment (start 183.4084 55.9008) (end 183.7883 56.2807) (width 0.2) (layer "B.Cu") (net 19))
 (segment (start 192.62 62.9813) (end 192.62 88) (width 0.2) (layer "B.Cu") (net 19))
 (segment (start 122.16 116.5) (end 131.92 116.5) (width 0.2) (layer "F.Cu") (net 3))
 (segment (start 164.68 77.54) (end 164.68 77.6875) (width 0.2) (layer "F.Cu") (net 3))
 (segment (start 171.5 77.54) (end 164.68 77.54) (width 0.2) (layer "F.Cu") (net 3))
 (segment (start 164.68 77.54) (end 137.88 77.54) (width 0.2) (layer "F.Cu") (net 3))
 (segment (start 137.88 77.54) (end 132 71.66) (width 0.2) (layer "F.Cu") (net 3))
 (via (at 164.68 77.6875) (size 0.6) (drill 0.3) (layers "F.Cu" "B.Cu") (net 3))
 (segment (start 130.322 101.66) (end 130.322 114.902) (width 0.2) (layer "B.Cu") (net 3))
 (segment (start 132 71.66) (end 132 99.982) (width 0.2) (layer "B.Cu") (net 3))
 (segment (start 153.1 56.665) (end 164.68 68.245) (width 0.2) (layer "B.Cu") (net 3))
 (segment (start 169.5 109.675) (end 168.6162 108.7912) (width 0.2) (layer "B.Cu") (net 3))
 (segment (start 164.68 77.6875) (end 164.68 88) (width 0.2) (layer "B.Cu") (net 3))
 (segment (start 168.6162 108.7912) (end 168.6162 80.4238) (width 0.2) (layer "B.Cu") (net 3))
 (segment (start 117.1275 111.4675) (end 122.16 116.5) (width 0.2) (layer "B.Cu") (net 3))
 (segment (start 132 99.982) (end 130.322 101.66) (width 0.2) (layer "B.Cu") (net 3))
 (segment (start 130.322 114.902) (end 131.92 116.5) (width 0.2) (layer "B.Cu") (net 3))
 (segment (start 117.1275 109.28) (end 117.1275 111.4675) (width 0.2) (layer "B.Cu") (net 3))
 (segment (start 164.68 68.245) (end 164.68 77.6875) (width 0.2) (layer "B.Cu") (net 3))
 (segment (start 168.6162 80.4238) (end 171.5 77.54) (width 0.2) (layer "B.Cu") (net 3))
 (segment (start 130.322 101.66) (end 129.8275 101.66) (width 0.2) (layer "B.Cu") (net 3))
 (segment (start 180.2316 109.675) (end 186.4383 103.4683) (width 0.2) (layer "F.Cu") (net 16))
 (segment (start 171.5 109.675) (end 180.2316 109.675) (width 0.2) (layer "F.Cu") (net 16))
 (segment (start 187.54 103.24) (end 186.4383 103.24) (width 0.2) (layer "F.Cu") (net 16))
 (segment (start 186.4383 103.4683) (end 186.4383 103.24) (width 0.2) (layer "F.Cu") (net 16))
 (segment (start 153.1 100.3062) (end 157.5503 100.3062) (width 0.2) (layer "F.Cu") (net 18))
 (segment (start 191.5183 103.1023) (end 188.7222 100.3062) (width 0.2) (layer "F.Cu") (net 18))
 (segment (start 188.7222 100.3062) (end 157.5503 100.3062) (width 0.2) (layer "F.Cu") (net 18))
 (segment (start 191.5183 103.24) (end 191.5183 103.1023) (width 0.2) (layer "F.Cu") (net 18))
 (segment (start 157.5503 100.3062) (end 153.1 100.3062) (width 0.2) (layer "F.Cu") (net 18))
 (segment (start 192.62 103.24) (end 191.5183 103.24) (width 0.2) (layer "F.Cu") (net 18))
 (via (at 157.5503 100.3062) (size 0.6) (drill 0.3) (layers "F.Cu" "B.Cu") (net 18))
 (segment (start 153.1 100.3062) (end 157.5503 100.3062) (width 0.2) (layer "B.Cu") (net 18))
 (segment (start 153.1 95.8559) (end 153.1 66.825) (width 0.2) (layer "B.Cu") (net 18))
 (segment (start 157.5503 100.3062) (end 153.1 100.3062) (width 0.2) (layer "B.Cu") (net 18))
 (segment (start 157.5503 100.3062) (end 153.1 95.8559) (width 0.2) (layer "B.Cu") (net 18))
 (segment (start 152.7387 60.475) (end 151.903 61.3107) (width 0.2) (layer "F.Cu") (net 32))
 (segment (start 151.903 63.088) (end 153.1 64.285) (width 0.2) (layer "F.Cu") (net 32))
 (segment (start 151.903 61.3107) (end 151.903 63.088) (width 0.2) (layer "F.Cu") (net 32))
 (segment (start 168 58.92) (end 166.445 60.475) (width 0.2) (layer "F.Cu") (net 32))
 (segment (start 166.445 60.475) (end 152.7387 60.475) (width 0.2) (layer "F.Cu") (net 32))
 (segment (start 167.42 54.5) (end 168 55.08) (width 0.2) (layer "B.Cu") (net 32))
 (segment (start 168 55.08) (end 168 58.92) (width 0.2) (layer "B.Cu") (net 32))
 (segment (start 120 58) (end 112.5 65.5) (width 0.2) (layer "F.Cu") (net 31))
 (segment (start 112.5 65.5) (end 108.5 65.5) (width 0.2) (layer "F.Cu") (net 31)))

